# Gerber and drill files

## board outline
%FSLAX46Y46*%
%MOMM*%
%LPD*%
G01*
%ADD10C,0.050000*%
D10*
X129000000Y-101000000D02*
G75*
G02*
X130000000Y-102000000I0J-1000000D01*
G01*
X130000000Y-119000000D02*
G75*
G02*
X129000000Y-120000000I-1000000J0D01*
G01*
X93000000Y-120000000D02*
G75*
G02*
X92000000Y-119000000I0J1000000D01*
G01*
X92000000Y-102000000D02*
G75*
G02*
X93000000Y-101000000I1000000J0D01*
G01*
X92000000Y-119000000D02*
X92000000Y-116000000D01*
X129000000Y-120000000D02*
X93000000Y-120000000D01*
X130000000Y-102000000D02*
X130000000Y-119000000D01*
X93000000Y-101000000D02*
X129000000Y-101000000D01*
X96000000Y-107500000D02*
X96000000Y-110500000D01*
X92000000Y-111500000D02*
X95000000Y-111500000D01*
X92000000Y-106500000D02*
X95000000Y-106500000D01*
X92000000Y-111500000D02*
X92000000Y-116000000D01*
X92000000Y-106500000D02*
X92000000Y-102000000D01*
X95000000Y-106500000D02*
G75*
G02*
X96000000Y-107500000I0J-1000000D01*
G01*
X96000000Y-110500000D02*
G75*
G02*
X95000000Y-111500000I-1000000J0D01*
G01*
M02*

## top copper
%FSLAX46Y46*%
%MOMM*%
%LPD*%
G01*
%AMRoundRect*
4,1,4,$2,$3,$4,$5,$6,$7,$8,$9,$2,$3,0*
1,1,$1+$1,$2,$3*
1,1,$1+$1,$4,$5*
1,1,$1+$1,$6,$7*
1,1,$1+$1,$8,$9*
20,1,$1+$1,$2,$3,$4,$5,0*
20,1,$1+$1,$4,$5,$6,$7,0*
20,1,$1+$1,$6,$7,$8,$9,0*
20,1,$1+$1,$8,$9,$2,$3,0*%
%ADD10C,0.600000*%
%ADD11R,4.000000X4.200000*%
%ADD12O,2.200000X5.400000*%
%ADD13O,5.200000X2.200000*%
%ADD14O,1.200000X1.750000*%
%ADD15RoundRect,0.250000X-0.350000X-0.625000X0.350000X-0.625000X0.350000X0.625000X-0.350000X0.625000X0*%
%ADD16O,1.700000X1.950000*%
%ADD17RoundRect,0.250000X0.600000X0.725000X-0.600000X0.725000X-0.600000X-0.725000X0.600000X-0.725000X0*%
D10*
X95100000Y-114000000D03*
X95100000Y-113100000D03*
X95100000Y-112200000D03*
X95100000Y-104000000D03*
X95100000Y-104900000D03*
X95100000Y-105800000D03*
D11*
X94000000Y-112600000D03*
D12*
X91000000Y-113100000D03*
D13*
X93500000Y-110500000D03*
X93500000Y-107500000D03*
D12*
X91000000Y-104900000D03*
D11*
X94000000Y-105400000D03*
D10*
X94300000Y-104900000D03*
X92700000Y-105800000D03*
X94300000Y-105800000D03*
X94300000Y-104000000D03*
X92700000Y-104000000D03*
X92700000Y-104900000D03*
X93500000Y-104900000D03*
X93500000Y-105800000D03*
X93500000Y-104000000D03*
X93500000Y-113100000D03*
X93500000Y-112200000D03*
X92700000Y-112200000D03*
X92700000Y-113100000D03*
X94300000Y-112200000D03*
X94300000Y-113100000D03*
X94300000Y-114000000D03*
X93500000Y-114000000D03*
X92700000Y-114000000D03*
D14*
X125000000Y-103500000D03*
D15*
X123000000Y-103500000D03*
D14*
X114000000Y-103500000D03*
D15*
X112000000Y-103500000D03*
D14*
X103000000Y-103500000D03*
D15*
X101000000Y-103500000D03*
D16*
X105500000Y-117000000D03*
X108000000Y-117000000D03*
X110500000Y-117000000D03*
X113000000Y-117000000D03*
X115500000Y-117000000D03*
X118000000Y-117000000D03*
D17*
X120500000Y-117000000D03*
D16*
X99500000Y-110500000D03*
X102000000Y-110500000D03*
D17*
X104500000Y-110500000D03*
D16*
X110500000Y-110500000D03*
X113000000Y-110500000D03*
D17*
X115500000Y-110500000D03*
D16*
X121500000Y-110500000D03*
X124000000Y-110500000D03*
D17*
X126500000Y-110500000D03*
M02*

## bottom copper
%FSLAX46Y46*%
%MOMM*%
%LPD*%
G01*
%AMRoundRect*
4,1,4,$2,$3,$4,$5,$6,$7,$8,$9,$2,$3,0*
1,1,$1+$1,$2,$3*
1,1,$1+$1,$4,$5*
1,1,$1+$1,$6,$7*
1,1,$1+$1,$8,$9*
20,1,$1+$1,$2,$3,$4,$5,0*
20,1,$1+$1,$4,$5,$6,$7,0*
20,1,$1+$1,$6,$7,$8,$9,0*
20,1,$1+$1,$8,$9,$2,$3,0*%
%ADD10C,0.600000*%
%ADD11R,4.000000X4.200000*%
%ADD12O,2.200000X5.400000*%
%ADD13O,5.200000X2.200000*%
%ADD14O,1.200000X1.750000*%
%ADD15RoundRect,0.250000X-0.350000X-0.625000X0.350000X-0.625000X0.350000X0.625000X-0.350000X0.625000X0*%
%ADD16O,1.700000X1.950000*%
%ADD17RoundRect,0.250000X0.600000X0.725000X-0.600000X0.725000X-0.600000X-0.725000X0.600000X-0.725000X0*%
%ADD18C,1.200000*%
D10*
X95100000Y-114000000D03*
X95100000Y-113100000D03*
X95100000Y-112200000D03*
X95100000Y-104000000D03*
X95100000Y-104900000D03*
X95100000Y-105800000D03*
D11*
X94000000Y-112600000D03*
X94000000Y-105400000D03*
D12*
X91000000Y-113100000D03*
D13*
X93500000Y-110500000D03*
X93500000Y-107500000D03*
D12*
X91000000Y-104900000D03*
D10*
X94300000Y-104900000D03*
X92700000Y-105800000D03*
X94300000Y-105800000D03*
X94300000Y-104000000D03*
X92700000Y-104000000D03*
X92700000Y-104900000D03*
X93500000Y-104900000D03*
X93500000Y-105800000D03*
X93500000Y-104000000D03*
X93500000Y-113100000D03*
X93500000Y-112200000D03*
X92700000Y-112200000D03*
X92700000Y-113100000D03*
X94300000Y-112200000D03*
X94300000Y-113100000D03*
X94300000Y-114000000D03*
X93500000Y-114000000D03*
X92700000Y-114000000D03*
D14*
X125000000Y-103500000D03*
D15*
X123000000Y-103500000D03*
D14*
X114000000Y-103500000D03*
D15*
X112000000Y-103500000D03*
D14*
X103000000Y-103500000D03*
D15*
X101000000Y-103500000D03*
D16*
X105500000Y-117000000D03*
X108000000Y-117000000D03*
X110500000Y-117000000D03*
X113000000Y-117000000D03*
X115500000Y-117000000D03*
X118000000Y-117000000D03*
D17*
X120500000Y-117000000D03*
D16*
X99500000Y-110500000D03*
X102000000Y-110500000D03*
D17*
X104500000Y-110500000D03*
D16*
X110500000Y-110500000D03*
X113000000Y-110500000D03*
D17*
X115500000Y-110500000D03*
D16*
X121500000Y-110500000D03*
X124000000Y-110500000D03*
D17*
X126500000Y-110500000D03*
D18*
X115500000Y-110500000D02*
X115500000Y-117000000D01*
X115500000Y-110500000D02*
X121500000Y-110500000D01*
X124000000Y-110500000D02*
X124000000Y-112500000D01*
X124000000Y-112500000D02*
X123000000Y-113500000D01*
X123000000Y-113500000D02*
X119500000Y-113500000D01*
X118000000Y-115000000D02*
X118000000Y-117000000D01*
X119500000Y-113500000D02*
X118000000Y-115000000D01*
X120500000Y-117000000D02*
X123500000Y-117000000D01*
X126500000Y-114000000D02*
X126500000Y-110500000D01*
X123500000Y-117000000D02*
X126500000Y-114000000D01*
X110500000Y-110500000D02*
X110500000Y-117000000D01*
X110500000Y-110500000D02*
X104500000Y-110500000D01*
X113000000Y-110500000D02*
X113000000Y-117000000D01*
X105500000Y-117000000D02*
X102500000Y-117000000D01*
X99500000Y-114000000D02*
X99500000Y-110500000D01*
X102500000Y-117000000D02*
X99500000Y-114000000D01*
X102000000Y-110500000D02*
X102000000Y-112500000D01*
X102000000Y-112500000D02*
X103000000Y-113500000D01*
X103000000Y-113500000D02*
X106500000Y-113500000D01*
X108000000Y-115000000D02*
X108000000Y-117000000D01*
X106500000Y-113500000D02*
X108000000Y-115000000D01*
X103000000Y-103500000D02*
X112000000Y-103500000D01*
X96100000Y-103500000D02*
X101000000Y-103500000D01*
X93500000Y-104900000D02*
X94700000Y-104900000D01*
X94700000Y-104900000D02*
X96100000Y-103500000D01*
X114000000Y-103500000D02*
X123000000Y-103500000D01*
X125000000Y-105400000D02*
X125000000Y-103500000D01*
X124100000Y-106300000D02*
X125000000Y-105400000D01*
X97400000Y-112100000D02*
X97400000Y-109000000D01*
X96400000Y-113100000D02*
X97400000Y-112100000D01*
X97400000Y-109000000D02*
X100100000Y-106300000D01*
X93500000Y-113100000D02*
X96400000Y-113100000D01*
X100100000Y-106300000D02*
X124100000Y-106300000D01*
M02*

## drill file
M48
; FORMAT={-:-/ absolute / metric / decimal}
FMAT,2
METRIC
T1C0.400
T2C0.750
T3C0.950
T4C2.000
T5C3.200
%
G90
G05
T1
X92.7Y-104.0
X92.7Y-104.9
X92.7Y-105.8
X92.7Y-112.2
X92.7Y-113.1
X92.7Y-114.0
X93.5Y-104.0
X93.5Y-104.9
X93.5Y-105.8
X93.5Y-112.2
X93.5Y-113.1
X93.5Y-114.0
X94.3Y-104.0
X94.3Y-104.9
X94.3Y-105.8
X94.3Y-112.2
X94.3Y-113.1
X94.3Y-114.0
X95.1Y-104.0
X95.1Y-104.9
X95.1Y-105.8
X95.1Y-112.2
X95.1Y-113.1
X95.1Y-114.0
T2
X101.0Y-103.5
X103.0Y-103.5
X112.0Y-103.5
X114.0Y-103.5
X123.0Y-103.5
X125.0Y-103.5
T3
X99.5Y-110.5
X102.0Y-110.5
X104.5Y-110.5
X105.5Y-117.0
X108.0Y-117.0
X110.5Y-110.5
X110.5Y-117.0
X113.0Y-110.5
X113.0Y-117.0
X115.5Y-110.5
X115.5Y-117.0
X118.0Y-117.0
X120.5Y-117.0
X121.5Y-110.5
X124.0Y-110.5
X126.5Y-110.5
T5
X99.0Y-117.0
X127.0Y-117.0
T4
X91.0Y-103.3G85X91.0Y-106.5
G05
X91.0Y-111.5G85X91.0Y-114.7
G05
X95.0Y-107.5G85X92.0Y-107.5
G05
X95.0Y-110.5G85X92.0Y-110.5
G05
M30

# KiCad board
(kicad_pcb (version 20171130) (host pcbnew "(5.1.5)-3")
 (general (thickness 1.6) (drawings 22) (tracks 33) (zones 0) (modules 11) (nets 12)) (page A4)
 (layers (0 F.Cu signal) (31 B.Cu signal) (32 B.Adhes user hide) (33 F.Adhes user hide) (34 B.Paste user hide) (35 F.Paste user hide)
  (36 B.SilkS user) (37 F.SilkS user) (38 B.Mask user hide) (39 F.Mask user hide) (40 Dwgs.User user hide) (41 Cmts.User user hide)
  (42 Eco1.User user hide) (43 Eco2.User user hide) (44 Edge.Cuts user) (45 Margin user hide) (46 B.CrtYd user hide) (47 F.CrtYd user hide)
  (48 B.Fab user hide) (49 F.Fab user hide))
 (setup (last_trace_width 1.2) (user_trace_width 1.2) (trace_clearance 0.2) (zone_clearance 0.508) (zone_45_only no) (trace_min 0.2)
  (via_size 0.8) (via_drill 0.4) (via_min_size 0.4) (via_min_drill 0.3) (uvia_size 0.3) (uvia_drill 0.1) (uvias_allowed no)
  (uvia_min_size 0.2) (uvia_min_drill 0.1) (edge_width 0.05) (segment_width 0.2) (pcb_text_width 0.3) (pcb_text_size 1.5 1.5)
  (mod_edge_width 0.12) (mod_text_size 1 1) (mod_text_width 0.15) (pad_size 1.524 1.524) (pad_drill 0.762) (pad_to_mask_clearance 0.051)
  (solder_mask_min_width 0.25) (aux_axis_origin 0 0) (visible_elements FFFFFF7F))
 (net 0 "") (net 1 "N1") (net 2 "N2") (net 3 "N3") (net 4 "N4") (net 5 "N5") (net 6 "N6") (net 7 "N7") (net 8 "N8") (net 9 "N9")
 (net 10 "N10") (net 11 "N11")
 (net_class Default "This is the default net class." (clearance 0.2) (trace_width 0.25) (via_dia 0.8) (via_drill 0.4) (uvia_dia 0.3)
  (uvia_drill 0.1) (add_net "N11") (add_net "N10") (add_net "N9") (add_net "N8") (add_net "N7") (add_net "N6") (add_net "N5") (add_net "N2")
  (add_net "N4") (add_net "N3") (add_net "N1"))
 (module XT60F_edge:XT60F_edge (layer F.Cu) (at 92 109 270)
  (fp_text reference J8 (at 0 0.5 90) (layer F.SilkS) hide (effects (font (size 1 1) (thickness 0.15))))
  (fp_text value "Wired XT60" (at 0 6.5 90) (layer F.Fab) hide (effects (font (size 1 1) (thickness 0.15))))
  (fp_line (start -1.5 -4) (end 1.5 -4) (layer Edge.Cuts) (width 0.05))
  (fp_line (start 2.5 0) (end 2.5 -3) (layer Edge.Cuts) (width 0.05))
  (fp_line (start -2.5 0) (end -2.5 -3) (layer Edge.Cuts) (width 0.05))
  (fp_line (start 2.5 0) (end 7 0) (layer Edge.Cuts) (width 0.05))
  (fp_line (start -2.5 0) (end -7 0) (layer Edge.Cuts) (width 0.05))
  (fp_arc (start -1.5 -3) (end -1.5 -4) (angle -90) (layer Edge.Cuts) (width 0.05))
  (fp_arc (start 1.5 -3) (end 2.5 -3) (angle -90) (layer Edge.Cuts) (width 0.05))
  (pad 2 thru_hole circle (at 5 -3.1 270) (size 0.6 0.6) (drill 0.4) (layers *.Cu *.Mask) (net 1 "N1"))
  (pad 2 thru_hole circle (at 4.1 -3.1 270) (size 0.6 0.6) (drill 0.4) (layers *.Cu *.Mask) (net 1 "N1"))
  (pad 2 thru_hole circle (at 3.2 -3.1 270) (size 0.6 0.6) (drill 0.4) (layers *.Cu *.Mask) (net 1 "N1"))
  (pad 1 thru_hole circle (at -5 -3.1 270) (size 0.6 0.6) (drill 0.4) (layers *.Cu *.Mask) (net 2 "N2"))
  (pad 1 thru_hole circle (at -4.1 -3.1 270) (size 0.6 0.6) (drill 0.4) (layers *.Cu *.Mask) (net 2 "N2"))
  (pad 1 thru_hole circle (at -3.2 -3.1 270) (size 0.6 0.6) (drill 0.4) (layers *.Cu *.Mask) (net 2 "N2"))
  (pad 2 connect rect (at 3.6 -2 270) (size 4.2 4) (layers B.Cu F.Mask) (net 1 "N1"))
  (pad 2 connect rect (at 3.6 -2 270) (size 4.2 4) (layers F.Cu F.Mask) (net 1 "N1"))
  (pad 1 connect rect (at -3.6 -2 270) (size 4.2 4) (layers B.Cu F.Mask) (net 2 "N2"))
  (pad 2 thru_hole oval (at 4.1 1 270) (size 5.4 2.2) (drill oval 5.2 2) (layers *.Cu *.Mask) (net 1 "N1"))
  (pad 2 thru_hole oval (at 1.5 -1.5 270) (size 2.2 5.2) (drill oval 2 5) (layers *.Cu *.Mask) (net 1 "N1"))
  (pad 1 thru_hole oval (at -1.5 -1.5 270) (size 2.2 5.2) (drill oval 2 5) (layers *.Cu *.Mask) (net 2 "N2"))
  (pad 1 thru_hole oval (at -4.1 1 270) (size 5.4 2.2) (drill oval 5.2 2) (layers *.Cu *.Mask) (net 2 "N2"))
  (pad 1 connect rect (at -3.6 -2 270) (size 4.2 4) (layers F.Cu F.Mask) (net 2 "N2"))
  (pad 1 thru_hole circle (at -4.1 -2.3 270) (size 0.6 0.6) (drill 0.4) (layers *.Cu *.Mask) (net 2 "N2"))
  (pad 1 thru_hole circle (at -3.2 -0.7 270) (size 0.6 0.6) (drill 0.4) (layers *.Cu *.Mask) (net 2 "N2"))
  (pad 1 thru_hole circle (at -3.2 -2.3 270) (size 0.6 0.6) (drill 0.4) (layers *.Cu *.Mask) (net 2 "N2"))
  (pad 1 thru_hole circle (at -5 -2.3 270) (size 0.6 0.6) (drill 0.4) (layers *.Cu *.Mask) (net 2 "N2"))
  (pad 1 thru_hole circle (at -5 -0.7 270) (size 0.6 0.6) (drill 0.4) (layers *.Cu *.Mask) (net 2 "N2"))
  (pad 1 thru_hole circle (at -4.1 -0.7 270) (size 0.6 0.6) (drill 0.4) (layers *.Cu *.Mask) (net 2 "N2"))
  (pad 1 thru_hole circle (at -4.1 -1.5 270) (size 0.6 0.6) (drill 0.4) (layers *.Cu *.Mask) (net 2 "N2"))
  (pad 1 thru_hole circle (at -3.2 -1.5 270) (size 0.6 0.6) (drill 0.4) (layers *.Cu *.Mask) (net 2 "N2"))
  (pad 1 thru_hole circle (at -5 -1.5 270) (size 0.6 0.6) (drill 0.4) (layers *.Cu *.Mask) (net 2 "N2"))
  (pad 2 thru_hole circle (at 4.1 -1.5 270) (size 0.6 0.6) (drill 0.4) (layers *.Cu *.Mask) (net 1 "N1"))
  (pad 2 thru_hole circle (at 3.2 -1.5 270) (size 0.6 0.6) (drill 0.4) (layers *.Cu *.Mask) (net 1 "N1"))
  (pad 2 thru_hole circle (at 3.2 -0.7 270) (size 0.6 0.6) (drill 0.4) (layers *.Cu *.Mask) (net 1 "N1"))
  (pad 2 thru_hole circle (at 4.1 -0.7 270) (size 0.6 0.6) (drill 0.4) (layers *.Cu *.Mask) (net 1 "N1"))
  (pad 2 thru_hole circle (at 3.2 -2.3 270) (size 0.6 0.6) (drill 0.4) (layers *.Cu *.Mask) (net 1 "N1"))
  (pad 2 thru_hole circle (at 4.1 -2.3 270) (size 0.6 0.6) (drill 0.4) (layers *.Cu *.Mask) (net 1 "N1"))
  (pad 2 thru_hole circle (at 5 -2.3 270) (size 0.6 0.6) (drill 0.4) (layers *.Cu *.Mask) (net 1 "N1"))
  (pad 2 thru_hole circle (at 5 -1.5 270) (size 0.6 0.6) (drill 0.4) (layers *.Cu *.Mask) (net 1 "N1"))
  (pad 2 thru_hole circle (at 5 -0.7 270) (size 0.6 0.6) (drill 0.4) (layers *.Cu *.Mask) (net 1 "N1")))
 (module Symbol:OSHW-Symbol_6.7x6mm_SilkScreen (layer B.Cu) (at 118.5 104.5 180)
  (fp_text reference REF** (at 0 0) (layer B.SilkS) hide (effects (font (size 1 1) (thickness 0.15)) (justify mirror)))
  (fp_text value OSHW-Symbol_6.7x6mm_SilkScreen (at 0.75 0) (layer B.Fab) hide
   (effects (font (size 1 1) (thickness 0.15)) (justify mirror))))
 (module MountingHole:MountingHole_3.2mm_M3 (layer F.Cu) (at 127 117)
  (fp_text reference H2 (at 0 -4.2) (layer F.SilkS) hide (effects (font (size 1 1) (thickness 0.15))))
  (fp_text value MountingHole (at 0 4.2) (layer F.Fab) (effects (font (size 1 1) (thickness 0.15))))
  (pad 1 np_thru_hole circle (at 0 0) (size 3.2 3.2) (drill 3.2) (layers *.Cu *.Mask)))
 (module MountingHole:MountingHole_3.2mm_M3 (layer F.Cu) (at 99 117)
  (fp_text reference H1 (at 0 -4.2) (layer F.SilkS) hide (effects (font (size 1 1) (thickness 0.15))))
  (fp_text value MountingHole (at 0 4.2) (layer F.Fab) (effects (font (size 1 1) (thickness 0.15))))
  (pad 1 np_thru_hole circle (at 0 0) (size 3.2 3.2) (drill 3.2) (layers *.Cu *.Mask)))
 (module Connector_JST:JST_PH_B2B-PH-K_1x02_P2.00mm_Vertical (layer F.Cu) (at 123 103.5)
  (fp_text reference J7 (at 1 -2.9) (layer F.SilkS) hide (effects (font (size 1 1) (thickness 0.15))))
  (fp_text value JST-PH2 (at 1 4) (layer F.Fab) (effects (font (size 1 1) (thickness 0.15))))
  (pad 2 thru_hole oval (at 2 0) (size 1.2 1.75) (drill 0.75) (layers *.Cu *.Mask) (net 1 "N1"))
  (pad 1 thru_hole roundrect (at 0 0) (size 1.2 1.75) (drill 0.75) (layers *.Cu *.Mask) (roundrect_rratio 0.208333) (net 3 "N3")))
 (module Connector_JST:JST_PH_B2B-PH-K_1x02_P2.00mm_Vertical (layer F.Cu) (at 112 103.5)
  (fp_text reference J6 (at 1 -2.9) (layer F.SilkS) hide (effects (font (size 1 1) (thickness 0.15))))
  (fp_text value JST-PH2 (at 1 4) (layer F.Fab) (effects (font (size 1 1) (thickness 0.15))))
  (pad 2 thru_hole oval (at 2 0) (size 1.2 1.75) (drill 0.75) (layers *.Cu *.Mask) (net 3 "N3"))
  (pad 1 thru_hole roundrect (at 0 0) (size 1.2 1.75) (drill 0.75) (layers *.Cu *.Mask) (roundrect_rratio 0.208333) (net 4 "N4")))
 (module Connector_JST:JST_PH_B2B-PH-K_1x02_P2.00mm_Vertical (layer F.Cu) (at 101 103.5)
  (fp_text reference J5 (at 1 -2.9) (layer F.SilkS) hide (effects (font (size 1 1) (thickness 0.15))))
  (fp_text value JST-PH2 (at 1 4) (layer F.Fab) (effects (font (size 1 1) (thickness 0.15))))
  (pad 2 thru_hole oval (at 2 0) (size 1.2 1.75) (drill 0.75) (layers *.Cu *.Mask) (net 4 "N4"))
  (pad 1 thru_hole roundrect (at 0 0) (size 1.2 1.75) (drill 0.75) (layers *.Cu *.Mask) (roundrect_rratio 0.208333) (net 2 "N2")))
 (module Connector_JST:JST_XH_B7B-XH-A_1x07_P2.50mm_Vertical (layer F.Cu) (at 120.5 117 180)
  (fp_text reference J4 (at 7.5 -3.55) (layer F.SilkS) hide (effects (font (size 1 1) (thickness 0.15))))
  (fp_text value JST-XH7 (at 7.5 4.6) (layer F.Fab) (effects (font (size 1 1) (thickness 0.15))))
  (pad 7 thru_hole oval (at 15 0 180) (size 1.7 1.95) (drill 0.95) (layers *.Cu *.Mask) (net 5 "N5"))
  (pad 6 thru_hole oval (at 12.5 0 180) (size 1.7 1.95) (drill 0.95) (layers *.Cu *.Mask) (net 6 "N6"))
  (pad 5 thru_hole oval (at 10 0 180) (size 1.7 1.95) (drill 0.95) (layers *.Cu *.Mask) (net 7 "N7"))
  (pad 4 thru_hole oval (at 7.5 0 180) (size 1.7 1.95) (drill 0.95) (layers *.Cu *.Mask) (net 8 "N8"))
  (pad 3 thru_hole oval (at 5 0 180) (size 1.7 1.95) (drill 0.95) (layers *.Cu *.Mask) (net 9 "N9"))
  (pad 2 thru_hole oval (at 2.5 0 180) (size 1.7 1.95) (drill 0.95) (layers *.Cu *.Mask) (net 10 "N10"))
  (pad 1 thru_hole roundrect (at 0 0 180) (size 1.7 1.95) (drill 0.95) (layers *.Cu *.Mask) (roundrect_rratio 0.147059) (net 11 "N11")))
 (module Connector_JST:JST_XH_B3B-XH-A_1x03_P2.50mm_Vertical (layer F.Cu) (at 104.5 110.5 180)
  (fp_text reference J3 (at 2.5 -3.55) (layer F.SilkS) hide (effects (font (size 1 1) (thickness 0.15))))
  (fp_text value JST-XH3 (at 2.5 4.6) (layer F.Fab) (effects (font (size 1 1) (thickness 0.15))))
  (pad 3 thru_hole oval (at 5 0 180) (size 1.7 1.95) (drill 0.95) (layers *.Cu *.Mask) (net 5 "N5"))
  (pad 2 thru_hole oval (at 2.5 0 180) (size 1.7 1.95) (drill 0.95) (layers *.Cu *.Mask) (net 6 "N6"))
  (pad 1 thru_hole roundrect (at 0 0 180) (size 1.7 1.95) (drill 0.95) (layers *.Cu *.Mask) (roundrect_rratio 0.147059) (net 7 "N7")))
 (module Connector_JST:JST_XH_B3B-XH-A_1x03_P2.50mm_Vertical (layer F.Cu) (at 115.5 110.5 180)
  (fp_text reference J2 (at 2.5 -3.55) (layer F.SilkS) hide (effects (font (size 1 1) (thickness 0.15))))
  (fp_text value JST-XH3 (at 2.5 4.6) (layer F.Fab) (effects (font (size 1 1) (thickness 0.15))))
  (pad 3 thru_hole oval (at 5 0 180) (size 1.7 1.95) (drill 0.95) (layers *.Cu *.Mask) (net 7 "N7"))
  (pad 2 thru_hole oval (at 2.5 0 180) (size 1.7 1.95) (drill 0.95) (layers *.Cu *.Mask) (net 8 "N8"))
  (pad 1 thru_hole roundrect (at 0 0 180) (size 1.7 1.95) (drill 0.95) (layers *.Cu *.Mask) (roundrect_rratio 0.147059) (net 9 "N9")))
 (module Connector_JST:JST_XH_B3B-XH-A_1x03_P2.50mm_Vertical (layer F.Cu) (at 126.5 110.5 180)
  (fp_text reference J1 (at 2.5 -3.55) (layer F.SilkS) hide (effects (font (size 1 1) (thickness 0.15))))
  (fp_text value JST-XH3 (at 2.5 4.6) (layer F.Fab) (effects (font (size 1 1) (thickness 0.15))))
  (pad 3 thru_hole oval (at 5 0 180) (size 1.7 1.95) (drill 0.95) (layers *.Cu *.Mask) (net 9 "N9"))
  (pad 2 thru_hole oval (at 2.5 0 180) (size 1.7 1.95) (drill 0.95) (layers *.Cu *.Mask) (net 10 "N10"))
  (pad 1 thru_hole roundrect (at 0 0 180) (size 1.7 1.95) (drill 0.95) (layers *.Cu *.Mask) (roundrect_rratio 0.147059) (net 11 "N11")))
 (gr_arc (start 129 102) (end 130 102) (angle -90) (layer Edge.Cuts) (width 0.05))
 (gr_arc (start 129 119) (end 129 120) (angle -90) (layer Edge.Cuts) (width 0.05))
 (gr_arc (start 93 119) (end 92 119) (angle -90) (layer Edge.Cuts) (width 0.05))
 (gr_arc (start 93 102) (end 93 101) (angle -90) (layer Edge.Cuts) (width 0.05))
 (gr_line (start 92 119) (end 92 116) (layer Edge.Cuts) (width 0.05))
 (gr_line (start 129 120) (end 93 120) (layer Edge.Cuts) (width 0.05))
 (gr_line (start 130 102) (end 130 119) (layer Edge.Cuts) (width 0.05))
 (gr_line (start 93 101) (end 129 101) (layer Edge.Cuts) (width 0.05))
 (segment (start 115.5 110.5) (end 115.5 117) (width 1.2) (layer B.Cu) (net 9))
 (segment (start 115.5 110.5) (end 121.5 110.5) (width 1.2) (layer B.Cu) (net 9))
 (segment (start 124 110.5) (end 124 112.5) (width 1.2) (layer B.Cu) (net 10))
 (segment (start 124 112.5) (end 123 113.5) (width 1.2) (layer B.Cu) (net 10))
 (segment (start 123 113.5) (end 119.5 113.5) (width 1.2) (layer B.Cu) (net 10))
 (segment (start 118 115) (end 118 117) (width 1.2) (layer B.Cu) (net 10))
 (segment (start 119.5 113.5) (end 118 115) (width 1.2) (layer B.Cu) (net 10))
 (segment (start 120.5 117) (end 123.5 117) (width 1.2) (layer B.Cu) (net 11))
 (segment (start 126.5 114) (end 126.5 110.5) (width 1.2) (layer B.Cu) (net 11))
 (segment (start 123.5 117) (end 126.5 114) (width 1.2) (layer B.Cu) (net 11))
 (segment (start 110.5 110.5) (end 110.5 117) (width 1.2) (layer B.Cu) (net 7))
 (segment (start 110.5 110.5) (end 104.5 110.5) (width 1.2) (layer B.Cu) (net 7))
 (segment (start 113 110.5) (end 113 117) (width 1.2) (layer B.Cu) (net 8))
 (segment (start 105.5 117) (end 102.5 117) (width 1.2) (layer B.Cu) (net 5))
 (segment (start 99.5 114) (end 99.5 110.5) (width 1.2) (layer B.Cu) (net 5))
 (segment (start 102.5 117) (end 99.5 114) (width 1.2) (layer B.Cu) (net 5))
 (segment (start 102 110.5) (end 102 112.5) (width 1.2) (layer B.Cu) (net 6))
 (segment (start 102 112.5) (end 103 113.5) (width 1.2) (layer B.Cu) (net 6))
 (segment (start 103 113.5) (end 106.5 113.5) (width 1.2) (layer B.Cu) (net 6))
 (segment (start 108 115) (end 108 117) (width 1.2) (layer B.Cu) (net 6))
 (segment (start 106.5 113.5) (end 108 115) (width 1.2) (layer B.Cu) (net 6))
 (segment (start 103 103.5) (end 112 103.5) (width 1.2) (layer B.Cu) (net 4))
 (segment (start 96.1 103.5) (end 101 103.5) (width 1.2) (layer B.Cu) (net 2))
 (segment (start 93.5 104.9) (end 94.7 104.9) (width 1.2) (layer B.Cu) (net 2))
 (segment (start 94.7 104.9) (end 96.1 103.5) (width 1.2) (layer B.Cu) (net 2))
 (segment (start 114 103.5) (end 123 103.5) (width 1.2) (layer B.Cu) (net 3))
 (segment (start 125 105.4) (end 125 103.5) (width 1.2) (layer B.Cu) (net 1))
 (segment (start 124.1 106.3) (end 125 105.4) (width 1.2) (layer B.Cu) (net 1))
 (segment (start 97.4 112.1) (end 97.4 109) (width 1.2) (layer B.Cu) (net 1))
 (segment (start 96.4 113.1) (end 97.4 112.1) (width 1.2) (layer B.Cu) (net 1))
 (segment (start 97.4 109) (end 100.1 106.3) (width 1.2) (layer B.Cu) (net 1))
 (segment (start 93.5 113.1) (end 96.4 113.1) (width 1.2) (layer B.Cu) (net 1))
 (segment (start 100.1 106.3) (end 124.1 106.3) (width 1.2) (layer B.Cu) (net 1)))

